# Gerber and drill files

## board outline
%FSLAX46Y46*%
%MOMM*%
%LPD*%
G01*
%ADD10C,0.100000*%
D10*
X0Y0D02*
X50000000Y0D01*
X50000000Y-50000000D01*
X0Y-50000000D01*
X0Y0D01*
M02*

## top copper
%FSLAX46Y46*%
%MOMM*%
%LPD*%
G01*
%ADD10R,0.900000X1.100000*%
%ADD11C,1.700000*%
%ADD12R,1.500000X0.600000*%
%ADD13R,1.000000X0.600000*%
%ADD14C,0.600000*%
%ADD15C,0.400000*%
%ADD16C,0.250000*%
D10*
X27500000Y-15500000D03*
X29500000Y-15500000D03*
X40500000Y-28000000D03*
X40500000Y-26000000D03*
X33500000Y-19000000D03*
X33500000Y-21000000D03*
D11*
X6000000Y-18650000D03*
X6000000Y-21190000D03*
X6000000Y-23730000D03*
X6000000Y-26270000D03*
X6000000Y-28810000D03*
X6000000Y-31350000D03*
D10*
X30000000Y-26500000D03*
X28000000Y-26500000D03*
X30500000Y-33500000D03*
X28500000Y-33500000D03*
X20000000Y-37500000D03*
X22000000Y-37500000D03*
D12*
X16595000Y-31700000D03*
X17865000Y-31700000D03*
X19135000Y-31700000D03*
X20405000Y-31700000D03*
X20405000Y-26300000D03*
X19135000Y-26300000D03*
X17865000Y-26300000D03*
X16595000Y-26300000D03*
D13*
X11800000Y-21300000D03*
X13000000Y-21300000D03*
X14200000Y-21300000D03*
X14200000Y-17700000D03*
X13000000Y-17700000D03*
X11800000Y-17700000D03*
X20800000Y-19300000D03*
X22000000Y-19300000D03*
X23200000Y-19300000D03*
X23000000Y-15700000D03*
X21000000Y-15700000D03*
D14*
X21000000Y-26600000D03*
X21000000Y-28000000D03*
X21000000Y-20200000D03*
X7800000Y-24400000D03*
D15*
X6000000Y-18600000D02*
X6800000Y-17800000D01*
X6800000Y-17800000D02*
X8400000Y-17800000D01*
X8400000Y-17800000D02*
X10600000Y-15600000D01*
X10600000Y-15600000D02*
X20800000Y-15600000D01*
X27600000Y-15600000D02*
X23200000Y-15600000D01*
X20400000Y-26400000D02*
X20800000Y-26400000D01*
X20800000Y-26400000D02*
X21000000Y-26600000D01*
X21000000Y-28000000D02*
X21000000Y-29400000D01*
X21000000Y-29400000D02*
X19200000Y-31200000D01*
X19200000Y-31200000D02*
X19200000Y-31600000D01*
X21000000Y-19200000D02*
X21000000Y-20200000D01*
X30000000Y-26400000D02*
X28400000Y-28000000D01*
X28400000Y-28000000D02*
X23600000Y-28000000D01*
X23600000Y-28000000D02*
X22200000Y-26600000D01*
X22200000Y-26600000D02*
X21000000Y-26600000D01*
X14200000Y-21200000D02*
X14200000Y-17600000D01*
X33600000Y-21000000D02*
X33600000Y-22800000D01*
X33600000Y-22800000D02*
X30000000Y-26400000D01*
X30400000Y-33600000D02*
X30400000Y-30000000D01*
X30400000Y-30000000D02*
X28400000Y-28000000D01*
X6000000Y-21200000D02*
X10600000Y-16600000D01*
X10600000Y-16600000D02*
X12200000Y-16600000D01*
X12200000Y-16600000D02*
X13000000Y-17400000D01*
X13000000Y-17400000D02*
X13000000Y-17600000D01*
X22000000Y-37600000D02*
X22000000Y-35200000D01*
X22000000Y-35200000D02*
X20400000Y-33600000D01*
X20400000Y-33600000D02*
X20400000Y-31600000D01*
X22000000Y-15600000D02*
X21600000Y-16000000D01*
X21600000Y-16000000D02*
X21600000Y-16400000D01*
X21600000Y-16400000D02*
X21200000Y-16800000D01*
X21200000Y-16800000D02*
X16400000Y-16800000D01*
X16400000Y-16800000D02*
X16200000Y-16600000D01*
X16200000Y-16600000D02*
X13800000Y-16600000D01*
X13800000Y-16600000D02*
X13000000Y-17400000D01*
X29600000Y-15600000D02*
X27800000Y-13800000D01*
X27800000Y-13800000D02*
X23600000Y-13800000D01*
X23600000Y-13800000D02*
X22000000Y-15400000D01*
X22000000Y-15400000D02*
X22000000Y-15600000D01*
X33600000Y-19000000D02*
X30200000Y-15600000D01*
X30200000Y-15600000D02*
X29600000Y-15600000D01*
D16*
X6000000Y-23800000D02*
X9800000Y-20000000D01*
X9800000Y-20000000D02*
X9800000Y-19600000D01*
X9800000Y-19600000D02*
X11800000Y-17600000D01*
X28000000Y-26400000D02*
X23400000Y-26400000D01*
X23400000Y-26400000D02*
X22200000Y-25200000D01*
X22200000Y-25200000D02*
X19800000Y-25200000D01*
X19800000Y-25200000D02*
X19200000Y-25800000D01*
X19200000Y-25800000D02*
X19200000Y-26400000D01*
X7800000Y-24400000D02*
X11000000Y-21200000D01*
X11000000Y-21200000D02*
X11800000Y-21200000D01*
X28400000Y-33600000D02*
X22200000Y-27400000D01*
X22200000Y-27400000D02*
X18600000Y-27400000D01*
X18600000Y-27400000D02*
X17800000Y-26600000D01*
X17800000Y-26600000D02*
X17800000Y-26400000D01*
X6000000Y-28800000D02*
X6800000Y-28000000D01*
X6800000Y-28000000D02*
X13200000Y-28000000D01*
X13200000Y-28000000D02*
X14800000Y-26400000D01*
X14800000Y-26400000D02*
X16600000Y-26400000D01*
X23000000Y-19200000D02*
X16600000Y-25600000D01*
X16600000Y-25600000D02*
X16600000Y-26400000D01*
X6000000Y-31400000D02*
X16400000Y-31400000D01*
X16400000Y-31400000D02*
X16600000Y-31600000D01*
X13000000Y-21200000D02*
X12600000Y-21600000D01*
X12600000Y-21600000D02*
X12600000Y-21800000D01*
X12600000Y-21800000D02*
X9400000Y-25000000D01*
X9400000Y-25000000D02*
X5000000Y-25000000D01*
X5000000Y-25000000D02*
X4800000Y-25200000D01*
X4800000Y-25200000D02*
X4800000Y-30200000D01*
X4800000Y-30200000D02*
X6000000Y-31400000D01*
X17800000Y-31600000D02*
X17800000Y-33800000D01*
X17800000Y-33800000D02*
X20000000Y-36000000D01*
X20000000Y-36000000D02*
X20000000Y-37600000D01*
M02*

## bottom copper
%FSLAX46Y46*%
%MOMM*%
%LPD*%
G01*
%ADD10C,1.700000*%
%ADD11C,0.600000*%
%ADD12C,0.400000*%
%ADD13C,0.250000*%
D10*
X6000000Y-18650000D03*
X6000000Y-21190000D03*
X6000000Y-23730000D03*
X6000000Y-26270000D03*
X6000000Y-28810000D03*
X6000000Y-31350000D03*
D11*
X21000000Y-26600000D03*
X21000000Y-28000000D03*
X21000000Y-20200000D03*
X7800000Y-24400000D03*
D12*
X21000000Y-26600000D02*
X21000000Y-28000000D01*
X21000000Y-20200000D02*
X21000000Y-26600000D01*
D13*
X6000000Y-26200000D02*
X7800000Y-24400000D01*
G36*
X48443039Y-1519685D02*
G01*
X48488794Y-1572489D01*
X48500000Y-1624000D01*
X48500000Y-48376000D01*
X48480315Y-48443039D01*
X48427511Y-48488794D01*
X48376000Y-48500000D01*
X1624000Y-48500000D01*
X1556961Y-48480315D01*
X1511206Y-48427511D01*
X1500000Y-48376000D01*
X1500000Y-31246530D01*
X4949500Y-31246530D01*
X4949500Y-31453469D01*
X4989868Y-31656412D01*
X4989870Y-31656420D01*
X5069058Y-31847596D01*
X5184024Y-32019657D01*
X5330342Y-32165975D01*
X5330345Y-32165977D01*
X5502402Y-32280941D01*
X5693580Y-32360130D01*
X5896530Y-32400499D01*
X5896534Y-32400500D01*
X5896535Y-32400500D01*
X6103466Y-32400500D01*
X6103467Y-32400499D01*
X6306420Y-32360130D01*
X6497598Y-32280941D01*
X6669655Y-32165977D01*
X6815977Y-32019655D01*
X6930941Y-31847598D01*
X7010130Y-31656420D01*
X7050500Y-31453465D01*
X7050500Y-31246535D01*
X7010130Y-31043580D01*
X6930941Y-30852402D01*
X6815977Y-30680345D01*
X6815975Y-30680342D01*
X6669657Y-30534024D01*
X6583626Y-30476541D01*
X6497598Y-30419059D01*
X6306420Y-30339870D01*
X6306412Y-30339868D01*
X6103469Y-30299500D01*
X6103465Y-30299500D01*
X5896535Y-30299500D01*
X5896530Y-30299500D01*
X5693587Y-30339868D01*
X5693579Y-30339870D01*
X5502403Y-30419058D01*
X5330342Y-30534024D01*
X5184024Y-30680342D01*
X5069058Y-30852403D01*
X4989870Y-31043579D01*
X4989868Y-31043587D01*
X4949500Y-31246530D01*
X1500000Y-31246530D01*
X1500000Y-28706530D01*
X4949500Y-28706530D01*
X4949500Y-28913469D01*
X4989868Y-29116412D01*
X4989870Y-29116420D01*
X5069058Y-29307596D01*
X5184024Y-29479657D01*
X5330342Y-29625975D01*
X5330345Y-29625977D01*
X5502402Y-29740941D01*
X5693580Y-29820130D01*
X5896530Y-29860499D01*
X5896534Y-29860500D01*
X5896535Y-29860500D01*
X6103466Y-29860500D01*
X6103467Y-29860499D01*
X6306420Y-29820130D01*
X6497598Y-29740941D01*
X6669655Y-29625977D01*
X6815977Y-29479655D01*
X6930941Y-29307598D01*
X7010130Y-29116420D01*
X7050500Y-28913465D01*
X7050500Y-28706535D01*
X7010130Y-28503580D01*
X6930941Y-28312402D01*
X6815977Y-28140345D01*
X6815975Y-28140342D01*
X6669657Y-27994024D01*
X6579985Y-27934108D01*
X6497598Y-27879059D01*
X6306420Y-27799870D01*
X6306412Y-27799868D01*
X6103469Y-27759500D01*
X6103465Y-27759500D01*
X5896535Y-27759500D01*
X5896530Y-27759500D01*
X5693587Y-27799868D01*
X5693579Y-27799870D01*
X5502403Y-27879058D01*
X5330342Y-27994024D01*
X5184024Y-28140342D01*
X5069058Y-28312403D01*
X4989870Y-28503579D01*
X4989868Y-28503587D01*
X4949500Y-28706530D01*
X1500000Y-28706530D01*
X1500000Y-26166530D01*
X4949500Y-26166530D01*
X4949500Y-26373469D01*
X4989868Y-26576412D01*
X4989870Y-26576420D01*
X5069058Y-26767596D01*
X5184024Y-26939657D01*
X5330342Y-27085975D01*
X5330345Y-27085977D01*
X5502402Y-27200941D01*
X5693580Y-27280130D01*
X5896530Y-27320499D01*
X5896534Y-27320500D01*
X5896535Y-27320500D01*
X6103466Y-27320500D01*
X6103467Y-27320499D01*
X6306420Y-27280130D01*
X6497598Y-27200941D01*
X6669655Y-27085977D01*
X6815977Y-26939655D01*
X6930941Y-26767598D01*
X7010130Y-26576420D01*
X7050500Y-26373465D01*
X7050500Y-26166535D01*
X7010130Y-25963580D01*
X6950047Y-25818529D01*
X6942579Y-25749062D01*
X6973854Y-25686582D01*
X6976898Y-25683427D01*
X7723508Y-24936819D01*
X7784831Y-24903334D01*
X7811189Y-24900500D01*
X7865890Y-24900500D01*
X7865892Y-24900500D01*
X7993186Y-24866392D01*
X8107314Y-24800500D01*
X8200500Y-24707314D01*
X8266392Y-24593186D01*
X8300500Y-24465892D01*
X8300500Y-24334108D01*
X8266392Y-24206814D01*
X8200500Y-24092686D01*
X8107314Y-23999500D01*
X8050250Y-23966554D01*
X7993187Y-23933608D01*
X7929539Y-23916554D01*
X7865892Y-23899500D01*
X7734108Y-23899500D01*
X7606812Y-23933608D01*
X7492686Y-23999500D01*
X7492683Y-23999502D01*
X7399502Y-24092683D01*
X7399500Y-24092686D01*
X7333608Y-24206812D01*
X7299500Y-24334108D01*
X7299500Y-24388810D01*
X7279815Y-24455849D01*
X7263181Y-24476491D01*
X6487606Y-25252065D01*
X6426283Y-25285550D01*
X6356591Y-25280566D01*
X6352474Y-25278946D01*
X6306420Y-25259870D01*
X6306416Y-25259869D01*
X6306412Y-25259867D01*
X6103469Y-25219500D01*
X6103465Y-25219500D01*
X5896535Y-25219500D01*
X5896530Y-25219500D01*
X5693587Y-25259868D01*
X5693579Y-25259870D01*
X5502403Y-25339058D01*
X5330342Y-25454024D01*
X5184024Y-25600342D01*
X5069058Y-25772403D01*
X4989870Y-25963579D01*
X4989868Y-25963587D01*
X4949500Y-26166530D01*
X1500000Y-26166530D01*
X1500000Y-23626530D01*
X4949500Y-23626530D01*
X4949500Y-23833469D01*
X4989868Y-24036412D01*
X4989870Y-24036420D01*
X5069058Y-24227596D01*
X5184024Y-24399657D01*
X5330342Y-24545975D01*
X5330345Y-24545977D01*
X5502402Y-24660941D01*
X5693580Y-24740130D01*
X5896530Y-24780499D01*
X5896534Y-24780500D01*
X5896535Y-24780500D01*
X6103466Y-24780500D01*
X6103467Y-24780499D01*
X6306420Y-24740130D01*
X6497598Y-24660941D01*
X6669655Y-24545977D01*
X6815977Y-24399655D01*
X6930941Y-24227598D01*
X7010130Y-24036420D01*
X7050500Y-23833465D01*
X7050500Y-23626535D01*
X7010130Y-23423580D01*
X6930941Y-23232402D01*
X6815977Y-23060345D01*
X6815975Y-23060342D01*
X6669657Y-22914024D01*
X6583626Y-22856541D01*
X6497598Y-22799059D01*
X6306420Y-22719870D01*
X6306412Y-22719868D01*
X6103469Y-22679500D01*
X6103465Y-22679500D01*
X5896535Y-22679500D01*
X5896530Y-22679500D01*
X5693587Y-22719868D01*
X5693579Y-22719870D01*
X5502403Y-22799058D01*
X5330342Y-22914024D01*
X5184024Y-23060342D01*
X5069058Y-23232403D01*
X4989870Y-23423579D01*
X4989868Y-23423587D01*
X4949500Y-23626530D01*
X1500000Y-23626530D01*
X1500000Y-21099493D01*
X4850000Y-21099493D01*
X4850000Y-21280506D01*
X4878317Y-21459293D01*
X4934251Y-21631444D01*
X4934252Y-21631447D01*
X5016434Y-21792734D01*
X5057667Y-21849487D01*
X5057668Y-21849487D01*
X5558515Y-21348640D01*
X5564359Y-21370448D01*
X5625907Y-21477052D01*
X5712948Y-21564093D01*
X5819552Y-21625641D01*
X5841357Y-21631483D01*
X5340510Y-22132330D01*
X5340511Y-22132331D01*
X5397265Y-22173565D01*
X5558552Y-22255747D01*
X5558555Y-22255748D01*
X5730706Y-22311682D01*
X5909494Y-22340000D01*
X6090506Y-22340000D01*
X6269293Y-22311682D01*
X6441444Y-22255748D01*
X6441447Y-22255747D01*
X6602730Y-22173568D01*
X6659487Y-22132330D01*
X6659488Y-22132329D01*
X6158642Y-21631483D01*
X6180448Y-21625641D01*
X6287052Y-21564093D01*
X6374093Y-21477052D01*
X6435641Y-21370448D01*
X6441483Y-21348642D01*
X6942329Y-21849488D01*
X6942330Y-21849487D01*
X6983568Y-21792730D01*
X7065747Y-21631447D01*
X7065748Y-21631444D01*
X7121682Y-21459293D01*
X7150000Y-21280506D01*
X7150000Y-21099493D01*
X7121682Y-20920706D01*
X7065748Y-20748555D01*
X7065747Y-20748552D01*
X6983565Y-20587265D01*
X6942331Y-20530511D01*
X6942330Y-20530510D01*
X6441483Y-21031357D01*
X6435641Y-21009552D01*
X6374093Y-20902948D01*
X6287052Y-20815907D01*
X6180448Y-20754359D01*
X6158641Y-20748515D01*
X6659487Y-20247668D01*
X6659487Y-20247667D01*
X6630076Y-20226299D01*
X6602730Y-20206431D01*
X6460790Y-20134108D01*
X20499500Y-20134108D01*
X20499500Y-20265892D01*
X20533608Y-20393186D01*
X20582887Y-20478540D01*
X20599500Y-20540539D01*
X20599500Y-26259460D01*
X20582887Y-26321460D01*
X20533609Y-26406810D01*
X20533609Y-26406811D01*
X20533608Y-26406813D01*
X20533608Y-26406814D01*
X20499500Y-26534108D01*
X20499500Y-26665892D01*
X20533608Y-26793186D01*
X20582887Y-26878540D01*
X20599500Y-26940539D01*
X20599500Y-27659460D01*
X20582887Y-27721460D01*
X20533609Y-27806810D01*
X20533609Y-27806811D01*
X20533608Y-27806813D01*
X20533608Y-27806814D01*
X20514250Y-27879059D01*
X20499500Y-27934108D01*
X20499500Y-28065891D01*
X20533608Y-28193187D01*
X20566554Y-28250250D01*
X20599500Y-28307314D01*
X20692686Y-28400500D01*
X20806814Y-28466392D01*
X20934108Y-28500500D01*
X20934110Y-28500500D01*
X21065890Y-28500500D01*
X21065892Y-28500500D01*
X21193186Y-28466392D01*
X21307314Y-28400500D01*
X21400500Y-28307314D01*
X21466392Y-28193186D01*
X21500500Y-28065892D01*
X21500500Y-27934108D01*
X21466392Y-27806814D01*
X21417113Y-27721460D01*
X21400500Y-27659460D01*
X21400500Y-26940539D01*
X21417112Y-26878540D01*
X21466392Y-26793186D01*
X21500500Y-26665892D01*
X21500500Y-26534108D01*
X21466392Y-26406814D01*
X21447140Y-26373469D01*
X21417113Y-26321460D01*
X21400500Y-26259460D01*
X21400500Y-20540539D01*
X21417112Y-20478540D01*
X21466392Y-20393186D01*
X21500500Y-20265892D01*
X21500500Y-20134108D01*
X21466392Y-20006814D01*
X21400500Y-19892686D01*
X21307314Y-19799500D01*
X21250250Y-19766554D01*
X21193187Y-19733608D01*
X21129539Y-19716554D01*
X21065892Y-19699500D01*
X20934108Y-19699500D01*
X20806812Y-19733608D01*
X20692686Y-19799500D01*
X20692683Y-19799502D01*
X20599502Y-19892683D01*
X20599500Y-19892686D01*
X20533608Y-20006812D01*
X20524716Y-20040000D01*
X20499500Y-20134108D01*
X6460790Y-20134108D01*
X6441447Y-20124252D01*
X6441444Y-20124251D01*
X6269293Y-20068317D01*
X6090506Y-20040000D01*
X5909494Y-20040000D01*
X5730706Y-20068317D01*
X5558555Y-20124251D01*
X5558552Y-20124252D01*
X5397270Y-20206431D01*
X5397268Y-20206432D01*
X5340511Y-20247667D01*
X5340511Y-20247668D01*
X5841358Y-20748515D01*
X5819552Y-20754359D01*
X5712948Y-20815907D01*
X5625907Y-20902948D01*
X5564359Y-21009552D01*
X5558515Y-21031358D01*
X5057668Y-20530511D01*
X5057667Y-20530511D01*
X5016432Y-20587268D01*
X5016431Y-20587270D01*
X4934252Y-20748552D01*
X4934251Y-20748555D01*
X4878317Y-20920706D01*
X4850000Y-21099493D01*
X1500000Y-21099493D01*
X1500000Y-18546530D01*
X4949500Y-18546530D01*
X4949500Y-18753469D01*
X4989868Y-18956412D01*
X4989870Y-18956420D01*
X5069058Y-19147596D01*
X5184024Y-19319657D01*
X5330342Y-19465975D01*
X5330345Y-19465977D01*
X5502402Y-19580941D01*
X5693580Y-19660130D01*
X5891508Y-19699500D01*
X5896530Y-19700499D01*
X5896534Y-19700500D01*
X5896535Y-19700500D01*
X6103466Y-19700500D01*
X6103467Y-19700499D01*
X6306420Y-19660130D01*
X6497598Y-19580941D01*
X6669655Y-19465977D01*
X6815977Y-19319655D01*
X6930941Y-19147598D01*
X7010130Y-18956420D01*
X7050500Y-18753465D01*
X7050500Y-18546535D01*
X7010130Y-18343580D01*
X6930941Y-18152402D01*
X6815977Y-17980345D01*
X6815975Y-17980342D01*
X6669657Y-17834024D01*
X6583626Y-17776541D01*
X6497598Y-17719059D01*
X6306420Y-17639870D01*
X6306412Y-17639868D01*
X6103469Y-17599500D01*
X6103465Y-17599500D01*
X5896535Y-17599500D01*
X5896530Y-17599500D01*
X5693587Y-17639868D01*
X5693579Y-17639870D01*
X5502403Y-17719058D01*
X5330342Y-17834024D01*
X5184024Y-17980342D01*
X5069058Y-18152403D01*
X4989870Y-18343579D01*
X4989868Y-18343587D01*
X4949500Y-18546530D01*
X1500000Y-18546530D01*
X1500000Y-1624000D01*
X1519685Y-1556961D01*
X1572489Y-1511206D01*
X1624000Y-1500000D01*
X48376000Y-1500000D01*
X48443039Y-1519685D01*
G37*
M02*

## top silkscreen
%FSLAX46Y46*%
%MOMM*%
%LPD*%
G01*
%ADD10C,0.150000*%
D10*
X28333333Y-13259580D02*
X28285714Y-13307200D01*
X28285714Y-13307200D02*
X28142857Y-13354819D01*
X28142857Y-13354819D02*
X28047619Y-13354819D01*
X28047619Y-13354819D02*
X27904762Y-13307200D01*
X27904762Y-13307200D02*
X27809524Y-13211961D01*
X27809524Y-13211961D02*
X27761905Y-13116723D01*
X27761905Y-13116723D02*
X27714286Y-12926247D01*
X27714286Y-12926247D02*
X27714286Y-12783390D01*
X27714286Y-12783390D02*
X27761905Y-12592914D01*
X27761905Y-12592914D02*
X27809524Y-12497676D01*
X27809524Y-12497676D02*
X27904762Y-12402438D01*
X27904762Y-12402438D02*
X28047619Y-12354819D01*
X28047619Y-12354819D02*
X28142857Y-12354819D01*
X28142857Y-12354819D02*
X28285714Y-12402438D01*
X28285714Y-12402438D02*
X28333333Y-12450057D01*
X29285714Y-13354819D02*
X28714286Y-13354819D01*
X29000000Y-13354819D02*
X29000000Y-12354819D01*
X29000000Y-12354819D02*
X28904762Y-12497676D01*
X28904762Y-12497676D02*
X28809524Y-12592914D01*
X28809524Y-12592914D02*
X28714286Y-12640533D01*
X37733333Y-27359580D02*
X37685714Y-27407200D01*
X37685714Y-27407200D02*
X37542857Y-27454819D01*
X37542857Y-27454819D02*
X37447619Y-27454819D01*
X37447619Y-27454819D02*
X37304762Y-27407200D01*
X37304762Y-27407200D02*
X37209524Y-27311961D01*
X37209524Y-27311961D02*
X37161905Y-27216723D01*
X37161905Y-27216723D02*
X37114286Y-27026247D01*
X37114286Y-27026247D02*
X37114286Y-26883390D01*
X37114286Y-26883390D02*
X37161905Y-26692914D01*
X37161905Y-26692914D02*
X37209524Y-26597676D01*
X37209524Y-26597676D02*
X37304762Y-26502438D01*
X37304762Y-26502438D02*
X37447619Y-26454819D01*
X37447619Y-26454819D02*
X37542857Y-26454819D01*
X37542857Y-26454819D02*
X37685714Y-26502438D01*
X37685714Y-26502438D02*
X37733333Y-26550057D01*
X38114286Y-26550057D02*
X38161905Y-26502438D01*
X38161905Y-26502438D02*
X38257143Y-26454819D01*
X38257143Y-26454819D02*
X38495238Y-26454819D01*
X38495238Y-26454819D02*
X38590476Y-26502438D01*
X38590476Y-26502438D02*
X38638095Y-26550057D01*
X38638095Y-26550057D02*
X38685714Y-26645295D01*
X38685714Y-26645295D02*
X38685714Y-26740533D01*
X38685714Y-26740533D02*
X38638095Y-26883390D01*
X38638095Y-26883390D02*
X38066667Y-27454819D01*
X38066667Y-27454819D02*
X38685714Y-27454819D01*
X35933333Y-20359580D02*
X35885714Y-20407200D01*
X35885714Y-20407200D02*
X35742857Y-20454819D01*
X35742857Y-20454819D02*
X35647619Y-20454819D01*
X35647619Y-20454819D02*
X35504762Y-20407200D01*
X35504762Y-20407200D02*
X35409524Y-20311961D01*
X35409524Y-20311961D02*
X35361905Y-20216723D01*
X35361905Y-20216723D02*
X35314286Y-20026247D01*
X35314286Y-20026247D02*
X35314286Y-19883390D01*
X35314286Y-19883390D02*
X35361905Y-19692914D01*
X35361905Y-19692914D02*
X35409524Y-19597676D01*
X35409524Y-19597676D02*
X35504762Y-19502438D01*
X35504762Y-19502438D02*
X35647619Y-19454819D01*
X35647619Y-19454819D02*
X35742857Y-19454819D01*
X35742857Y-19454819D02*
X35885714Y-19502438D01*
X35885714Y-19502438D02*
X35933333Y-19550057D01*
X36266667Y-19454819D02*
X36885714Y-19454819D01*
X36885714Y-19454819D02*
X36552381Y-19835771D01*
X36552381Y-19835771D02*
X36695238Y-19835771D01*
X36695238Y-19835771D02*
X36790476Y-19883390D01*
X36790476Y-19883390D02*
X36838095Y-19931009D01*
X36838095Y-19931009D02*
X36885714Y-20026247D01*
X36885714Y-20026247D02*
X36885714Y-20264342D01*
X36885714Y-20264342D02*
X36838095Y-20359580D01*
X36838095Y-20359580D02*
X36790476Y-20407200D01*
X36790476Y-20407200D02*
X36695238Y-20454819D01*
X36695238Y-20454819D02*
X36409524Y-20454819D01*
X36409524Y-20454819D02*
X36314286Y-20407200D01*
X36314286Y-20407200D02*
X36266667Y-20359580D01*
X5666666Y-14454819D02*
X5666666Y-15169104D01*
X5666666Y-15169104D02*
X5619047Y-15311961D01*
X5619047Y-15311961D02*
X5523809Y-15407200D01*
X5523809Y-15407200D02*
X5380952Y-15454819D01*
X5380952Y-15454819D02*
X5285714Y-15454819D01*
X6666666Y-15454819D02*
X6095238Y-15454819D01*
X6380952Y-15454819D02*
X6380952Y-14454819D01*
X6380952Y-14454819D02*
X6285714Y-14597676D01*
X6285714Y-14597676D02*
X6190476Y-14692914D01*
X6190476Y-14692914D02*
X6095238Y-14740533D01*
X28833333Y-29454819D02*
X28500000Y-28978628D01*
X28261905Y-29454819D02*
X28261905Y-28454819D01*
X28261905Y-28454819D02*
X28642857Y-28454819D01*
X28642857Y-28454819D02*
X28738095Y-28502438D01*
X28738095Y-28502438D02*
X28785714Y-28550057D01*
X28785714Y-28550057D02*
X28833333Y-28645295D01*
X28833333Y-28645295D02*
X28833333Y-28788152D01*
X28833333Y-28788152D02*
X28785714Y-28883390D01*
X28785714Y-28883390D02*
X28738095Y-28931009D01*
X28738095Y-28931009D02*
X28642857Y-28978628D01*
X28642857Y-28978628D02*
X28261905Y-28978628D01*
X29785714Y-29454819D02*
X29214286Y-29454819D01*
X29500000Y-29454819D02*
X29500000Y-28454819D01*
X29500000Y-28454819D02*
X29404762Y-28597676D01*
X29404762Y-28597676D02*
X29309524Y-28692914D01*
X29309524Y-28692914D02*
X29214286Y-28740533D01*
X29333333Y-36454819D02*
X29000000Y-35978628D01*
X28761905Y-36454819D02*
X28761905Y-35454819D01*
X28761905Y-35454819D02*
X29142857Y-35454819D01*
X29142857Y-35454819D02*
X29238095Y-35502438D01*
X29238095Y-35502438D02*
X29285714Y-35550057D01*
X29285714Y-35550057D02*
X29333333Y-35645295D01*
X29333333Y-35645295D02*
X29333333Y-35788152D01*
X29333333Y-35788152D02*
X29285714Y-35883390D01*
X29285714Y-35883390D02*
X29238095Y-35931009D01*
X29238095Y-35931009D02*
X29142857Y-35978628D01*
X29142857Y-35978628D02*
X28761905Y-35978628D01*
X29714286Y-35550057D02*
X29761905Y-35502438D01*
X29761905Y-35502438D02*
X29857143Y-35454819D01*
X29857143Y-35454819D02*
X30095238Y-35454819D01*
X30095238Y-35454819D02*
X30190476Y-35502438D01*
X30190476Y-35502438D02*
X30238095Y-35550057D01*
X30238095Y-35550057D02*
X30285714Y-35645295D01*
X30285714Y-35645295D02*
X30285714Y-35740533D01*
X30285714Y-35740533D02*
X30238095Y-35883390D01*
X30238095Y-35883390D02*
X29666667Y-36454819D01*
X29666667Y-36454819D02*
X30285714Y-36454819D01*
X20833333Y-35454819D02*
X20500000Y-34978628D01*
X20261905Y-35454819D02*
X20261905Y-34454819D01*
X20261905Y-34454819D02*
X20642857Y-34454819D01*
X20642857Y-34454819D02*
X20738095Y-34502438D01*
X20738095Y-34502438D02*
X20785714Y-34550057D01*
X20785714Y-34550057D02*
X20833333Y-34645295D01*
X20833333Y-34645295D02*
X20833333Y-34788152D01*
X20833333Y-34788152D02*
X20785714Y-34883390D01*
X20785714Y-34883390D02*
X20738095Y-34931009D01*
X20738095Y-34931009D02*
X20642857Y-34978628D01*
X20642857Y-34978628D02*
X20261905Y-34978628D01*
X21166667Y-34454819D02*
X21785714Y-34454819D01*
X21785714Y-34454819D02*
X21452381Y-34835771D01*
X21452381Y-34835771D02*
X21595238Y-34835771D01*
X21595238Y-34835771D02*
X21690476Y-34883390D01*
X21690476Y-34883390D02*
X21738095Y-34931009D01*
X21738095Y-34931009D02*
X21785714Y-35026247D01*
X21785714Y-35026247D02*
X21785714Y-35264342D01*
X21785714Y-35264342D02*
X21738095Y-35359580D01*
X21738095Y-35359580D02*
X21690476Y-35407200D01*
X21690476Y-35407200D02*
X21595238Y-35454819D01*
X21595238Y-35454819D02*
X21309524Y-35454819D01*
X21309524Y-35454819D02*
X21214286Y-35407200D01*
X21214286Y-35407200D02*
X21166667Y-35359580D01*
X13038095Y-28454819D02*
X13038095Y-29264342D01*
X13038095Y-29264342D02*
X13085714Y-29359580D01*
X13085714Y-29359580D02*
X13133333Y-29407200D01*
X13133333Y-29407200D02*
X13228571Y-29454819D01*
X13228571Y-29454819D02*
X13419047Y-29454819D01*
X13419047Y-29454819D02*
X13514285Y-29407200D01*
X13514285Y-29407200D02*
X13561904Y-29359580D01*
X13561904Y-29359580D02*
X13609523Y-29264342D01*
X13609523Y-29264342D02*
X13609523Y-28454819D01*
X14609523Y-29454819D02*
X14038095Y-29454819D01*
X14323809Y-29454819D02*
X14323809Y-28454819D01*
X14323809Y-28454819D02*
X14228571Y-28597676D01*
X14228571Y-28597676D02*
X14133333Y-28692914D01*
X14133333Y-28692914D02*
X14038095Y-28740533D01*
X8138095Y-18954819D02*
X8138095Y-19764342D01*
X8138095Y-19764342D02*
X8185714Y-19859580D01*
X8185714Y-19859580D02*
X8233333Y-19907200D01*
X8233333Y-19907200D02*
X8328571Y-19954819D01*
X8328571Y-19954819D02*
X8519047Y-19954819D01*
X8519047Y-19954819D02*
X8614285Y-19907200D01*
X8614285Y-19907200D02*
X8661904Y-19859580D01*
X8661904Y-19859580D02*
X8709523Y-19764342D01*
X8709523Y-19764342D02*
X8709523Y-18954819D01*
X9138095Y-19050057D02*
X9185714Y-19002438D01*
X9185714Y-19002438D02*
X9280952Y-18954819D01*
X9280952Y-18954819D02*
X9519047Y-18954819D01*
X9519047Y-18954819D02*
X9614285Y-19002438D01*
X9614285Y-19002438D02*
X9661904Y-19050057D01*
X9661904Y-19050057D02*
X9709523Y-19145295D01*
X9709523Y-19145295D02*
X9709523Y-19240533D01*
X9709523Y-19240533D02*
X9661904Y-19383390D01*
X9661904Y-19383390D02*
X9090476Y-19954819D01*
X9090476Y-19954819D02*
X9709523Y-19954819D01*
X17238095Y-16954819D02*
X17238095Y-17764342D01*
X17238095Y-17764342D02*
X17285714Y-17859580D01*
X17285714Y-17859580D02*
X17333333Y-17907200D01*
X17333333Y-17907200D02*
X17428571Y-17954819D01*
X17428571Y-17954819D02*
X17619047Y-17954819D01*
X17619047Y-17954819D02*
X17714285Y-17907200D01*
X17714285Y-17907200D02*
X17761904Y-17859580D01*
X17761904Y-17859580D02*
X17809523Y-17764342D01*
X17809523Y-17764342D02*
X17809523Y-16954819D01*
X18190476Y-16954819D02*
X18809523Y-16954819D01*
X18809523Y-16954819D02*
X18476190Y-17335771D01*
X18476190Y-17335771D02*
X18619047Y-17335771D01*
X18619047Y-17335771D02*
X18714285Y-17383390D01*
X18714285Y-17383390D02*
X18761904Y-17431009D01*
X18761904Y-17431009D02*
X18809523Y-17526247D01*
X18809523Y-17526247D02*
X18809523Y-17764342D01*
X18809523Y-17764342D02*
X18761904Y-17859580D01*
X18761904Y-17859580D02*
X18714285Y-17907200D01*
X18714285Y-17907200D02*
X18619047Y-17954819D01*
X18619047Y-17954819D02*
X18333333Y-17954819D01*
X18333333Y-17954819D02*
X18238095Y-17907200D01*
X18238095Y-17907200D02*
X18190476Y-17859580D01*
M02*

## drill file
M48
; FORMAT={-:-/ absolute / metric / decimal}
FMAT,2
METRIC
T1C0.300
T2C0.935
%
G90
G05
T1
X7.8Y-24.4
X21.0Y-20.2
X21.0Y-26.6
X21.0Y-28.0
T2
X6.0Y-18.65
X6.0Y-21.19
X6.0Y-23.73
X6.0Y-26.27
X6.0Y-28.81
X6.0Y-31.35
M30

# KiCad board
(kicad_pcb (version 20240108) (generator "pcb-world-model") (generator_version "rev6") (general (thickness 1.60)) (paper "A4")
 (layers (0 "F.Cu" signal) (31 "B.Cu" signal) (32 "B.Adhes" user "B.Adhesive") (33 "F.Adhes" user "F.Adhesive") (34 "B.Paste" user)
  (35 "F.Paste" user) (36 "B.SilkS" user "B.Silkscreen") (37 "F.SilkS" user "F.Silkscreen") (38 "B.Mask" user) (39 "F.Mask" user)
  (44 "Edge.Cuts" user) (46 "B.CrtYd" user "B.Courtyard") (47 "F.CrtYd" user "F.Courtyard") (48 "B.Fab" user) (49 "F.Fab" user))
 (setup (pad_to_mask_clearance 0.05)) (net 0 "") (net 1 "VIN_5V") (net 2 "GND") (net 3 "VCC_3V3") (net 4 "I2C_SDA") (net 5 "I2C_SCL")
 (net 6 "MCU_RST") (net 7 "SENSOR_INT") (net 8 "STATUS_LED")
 (gr_rect (start 0.0 0.0) (end 50.0000 50.0000) (stroke (width 0.1) (type default)) (fill none) (layer "Edge.Cuts"))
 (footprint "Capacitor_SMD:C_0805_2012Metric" (layer "F.Cu") (at 28.5000 15.5000 0)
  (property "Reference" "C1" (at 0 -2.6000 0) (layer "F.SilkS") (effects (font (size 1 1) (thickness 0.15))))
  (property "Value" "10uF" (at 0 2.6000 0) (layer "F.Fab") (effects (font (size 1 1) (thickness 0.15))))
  (pad "1" smd rect (at -1.0000 0.0000) (size 0.9000 1.1000) (layers "F.Cu" "F.Paste" "F.Mask") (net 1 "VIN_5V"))
  (pad "2" smd rect (at 1.0000 0.0000) (size 0.9000 1.1000) (layers "F.Cu" "F.Paste" "F.Mask") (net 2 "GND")))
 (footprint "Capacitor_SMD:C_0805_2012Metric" (layer "F.Cu") (at 40.5000 27.0000 90)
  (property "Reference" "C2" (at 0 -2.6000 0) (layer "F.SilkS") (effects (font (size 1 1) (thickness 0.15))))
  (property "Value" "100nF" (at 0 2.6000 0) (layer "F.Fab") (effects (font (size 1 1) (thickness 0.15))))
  (pad "1" smd rect (at -1.0000 0.0000) (size 0.9000 1.1000) (layers "F.Cu" "F.Paste" "F.Mask") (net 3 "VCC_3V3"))
  (pad "2" smd rect (at 1.0000 0.0000) (size 0.9000 1.1000) (layers "F.Cu" "F.Paste" "F.Mask") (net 2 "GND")))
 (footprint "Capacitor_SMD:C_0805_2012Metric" (layer "F.Cu") (at 33.5000 20.0000 270)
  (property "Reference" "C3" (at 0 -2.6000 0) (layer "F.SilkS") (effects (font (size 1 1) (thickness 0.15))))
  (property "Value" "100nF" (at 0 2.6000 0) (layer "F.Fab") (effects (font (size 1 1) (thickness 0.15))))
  (pad "1" smd rect (at -1.0000 0.0000) (size 0.9000 1.1000) (layers "F.Cu" "F.Paste" "F.Mask") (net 3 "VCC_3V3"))
  (pad "2" smd rect (at 1.0000 0.0000) (size 0.9000 1.1000) (layers "F.Cu" "F.Paste" "F.Mask") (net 2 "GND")))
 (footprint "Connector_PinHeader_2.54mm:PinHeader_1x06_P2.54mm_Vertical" (layer "F.Cu") (at 6.0000 25.0000 0) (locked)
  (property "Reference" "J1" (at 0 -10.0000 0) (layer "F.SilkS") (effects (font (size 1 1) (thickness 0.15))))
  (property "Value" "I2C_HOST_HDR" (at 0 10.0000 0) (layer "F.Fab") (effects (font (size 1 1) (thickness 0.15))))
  (pad "1" thru_hole circle (at 0.0000 -6.3500) (size 1.7000 1.7000) (drill 0.9350) (layers "*.Cu" "*.Mask") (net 1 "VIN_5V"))
  (pad "2" thru_hole circle (at 0.0000 -3.8100) (size 1.7000 1.7000) (drill 0.9350) (layers "*.Cu" "*.Mask") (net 2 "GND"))
  (pad "3" thru_hole circle (at 0.0000 -1.2700) (size 1.7000 1.7000) (drill 0.9350) (layers "*.Cu" "*.Mask") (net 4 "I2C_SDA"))
  (pad "4" thru_hole circle (at 0.0000 1.2700) (size 1.7000 1.7000) (drill 0.9350) (layers "*.Cu" "*.Mask") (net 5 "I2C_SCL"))
  (pad "5" thru_hole circle (at 0.0000 3.8100) (size 1.7000 1.7000) (drill 0.9350) (layers "*.Cu" "*.Mask") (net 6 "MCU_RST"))
  (pad "6" thru_hole circle (at 0.0000 6.3500) (size 1.7000 1.7000) (drill 0.9350) (layers "*.Cu" "*.Mask") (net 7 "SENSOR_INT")))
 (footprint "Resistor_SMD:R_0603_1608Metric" (layer "F.Cu") (at 29.0000 26.5000 180)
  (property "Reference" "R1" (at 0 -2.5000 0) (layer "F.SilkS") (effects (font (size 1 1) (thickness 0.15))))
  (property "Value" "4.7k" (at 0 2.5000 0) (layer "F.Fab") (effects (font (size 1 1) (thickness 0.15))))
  (pad "1" smd rect (at -1.0000 0.0000) (size 0.9000 1.1000) (layers "F.Cu" "F.Paste" "F.Mask") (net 3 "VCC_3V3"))
  (pad "2" smd rect (at 1.0000 0.0000) (size 0.9000 1.1000) (layers "F.Cu" "F.Paste" "F.Mask") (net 4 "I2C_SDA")))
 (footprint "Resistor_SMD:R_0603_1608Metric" (layer "F.Cu") (at 29.5000 33.5000 180)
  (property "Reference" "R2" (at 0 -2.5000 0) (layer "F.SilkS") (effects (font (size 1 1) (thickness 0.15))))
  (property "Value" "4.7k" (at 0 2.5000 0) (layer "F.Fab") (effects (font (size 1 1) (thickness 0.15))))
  (pad "1" smd rect (at -1.0000 0.0000) (size 0.9000 1.1000) (layers "F.Cu" "F.Paste" "F.Mask") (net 3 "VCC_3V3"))
  (pad "2" smd rect (at 1.0000 0.0000) (size 0.9000 1.1000) (layers "F.Cu" "F.Paste" "F.Mask") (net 5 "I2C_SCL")))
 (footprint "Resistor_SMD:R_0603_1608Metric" (layer "F.Cu") (at 21.0000 37.5000 0)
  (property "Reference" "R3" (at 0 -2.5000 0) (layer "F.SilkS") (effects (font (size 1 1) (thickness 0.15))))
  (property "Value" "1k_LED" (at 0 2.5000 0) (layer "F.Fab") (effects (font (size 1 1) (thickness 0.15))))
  (pad "1" smd rect (at -1.0000 0.0000) (size 0.9000 1.1000) (layers "F.Cu" "F.Paste" "F.Mask") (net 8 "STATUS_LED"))
  (pad "2" smd rect (at 1.0000 0.0000) (size 0.9000 1.1000) (layers "F.Cu" "F.Paste" "F.Mask") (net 2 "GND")))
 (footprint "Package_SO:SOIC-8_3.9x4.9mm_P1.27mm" (layer "F.Cu") (at 18.5000 29.0000 90)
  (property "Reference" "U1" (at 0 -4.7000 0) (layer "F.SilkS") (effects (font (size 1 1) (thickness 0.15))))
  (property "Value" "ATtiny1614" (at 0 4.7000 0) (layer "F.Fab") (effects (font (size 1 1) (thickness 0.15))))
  (pad "1" smd rect (at -2.7000 -1.9050) (size 1.5000 0.6000) (layers "F.Cu" "F.Paste" "F.Mask") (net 3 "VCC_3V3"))
  (pad "2" smd rect (at -2.7000 -0.6350) (size 1.5000 0.6000) (layers "F.Cu" "F.Paste" "F.Mask") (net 4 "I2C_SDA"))
  (pad "3" smd rect (at -2.7000 0.6350) (size 1.5000 0.6000) (layers "F.Cu" "F.Paste" "F.Mask") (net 5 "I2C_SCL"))
  (pad "4" smd rect (at -2.7000 1.9050) (size 1.5000 0.6000) (layers "F.Cu" "F.Paste" "F.Mask") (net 6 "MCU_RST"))
  (pad "5" smd rect (at 2.7000 1.9050) (size 1.5000 0.6000) (layers "F.Cu" "F.Paste" "F.Mask") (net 7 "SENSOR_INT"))
  (pad "6" smd rect (at 2.7000 0.6350) (size 1.5000 0.6000) (layers "F.Cu" "F.Paste" "F.Mask") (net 8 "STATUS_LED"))
  (pad "7" smd rect (at 2.7000 -0.6350) (size 1.5000 0.6000) (layers "F.Cu" "F.Paste" "F.Mask") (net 3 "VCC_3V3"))
  (pad "8" smd rect (at 2.7000 -1.9050) (size 1.5000 0.6000) (layers "F.Cu" "F.Paste" "F.Mask") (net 2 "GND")))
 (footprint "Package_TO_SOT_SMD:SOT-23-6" (layer "F.Cu") (at 13.0000 19.5000 90)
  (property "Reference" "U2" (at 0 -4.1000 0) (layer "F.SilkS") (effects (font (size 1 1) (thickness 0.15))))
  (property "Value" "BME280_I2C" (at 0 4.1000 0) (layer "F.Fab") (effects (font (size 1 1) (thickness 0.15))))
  (pad "1" smd rect (at -1.8000 -1.2000) (size 1.0000 0.6000) (layers "F.Cu" "F.Paste" "F.Mask") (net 3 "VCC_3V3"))
  (pad "2" smd rect (at -1.8000 0.0000) (size 1.0000 0.6000) (layers "F.Cu" "F.Paste" "F.Mask") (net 2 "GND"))
  (pad "3" smd rect (at -1.8000 1.2000) (size 1.0000 0.6000) (layers "F.Cu" "F.Paste" "F.Mask") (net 4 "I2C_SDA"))
  (pad "4" smd rect (at 1.8000 1.2000) (size 1.0000 0.6000) (layers "F.Cu" "F.Paste" "F.Mask") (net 5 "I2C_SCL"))
  (pad "5" smd rect (at 1.8000 0.0000) (size 1.0000 0.6000) (layers "F.Cu" "F.Paste" "F.Mask") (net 7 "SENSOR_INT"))
  (pad "6" smd rect (at 1.8000 -1.2000) (size 1.0000 0.6000) (layers "F.Cu" "F.Paste" "F.Mask") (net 3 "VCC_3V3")))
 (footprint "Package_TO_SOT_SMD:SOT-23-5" (layer "F.Cu") (at 22.0000 17.5000 90)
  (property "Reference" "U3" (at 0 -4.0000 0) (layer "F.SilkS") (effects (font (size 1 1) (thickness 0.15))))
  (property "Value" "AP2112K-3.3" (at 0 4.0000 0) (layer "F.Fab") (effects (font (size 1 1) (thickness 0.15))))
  (pad "1" smd rect (at -1.8000 -1.2000) (size 1.0000 0.6000) (layers "F.Cu" "F.Paste" "F.Mask") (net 1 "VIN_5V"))
  (pad "2" smd rect (at -1.8000 0.0000) (size 1.0000 0.6000) (layers "F.Cu" "F.Paste" "F.Mask") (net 2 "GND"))
  (pad "3" smd rect (at -1.8000 1.2000) (size 1.0000 0.6000) (layers "F.Cu" "F.Paste" "F.Mask") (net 1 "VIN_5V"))
  (pad "4" smd rect (at 1.8000 1.0000) (size 1.0000 0.6000) (layers "F.Cu" "F.Paste" "F.Mask") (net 3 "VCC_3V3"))
  (pad "5" smd rect (at 1.8000 -1.0000) (size 1.0000 0.6000) (layers "F.Cu" "F.Paste" "F.Mask") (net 6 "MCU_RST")))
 (segment (start 6.0000 18.6000) (end 6.8000 17.8000) (width 0.4000) (layer "F.Cu") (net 1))
 (segment (start 6.8000 17.8000) (end 8.4000 17.8000) (width 0.4000) (layer "F.Cu") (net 1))
 (segment (start 8.4000 17.8000) (end 10.6000 15.6000) (width 0.4000) (layer "F.Cu") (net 1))
 (segment (start 10.6000 15.6000) (end 20.8000 15.6000) (width 0.4000) (layer "F.Cu") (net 1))
 (segment (start 27.6000 15.6000) (end 23.2000 15.6000) (width 0.4000) (layer "F.Cu") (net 1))
 (segment (start 20.4000 26.4000) (end 20.8000 26.4000) (width 0.4000) (layer "F.Cu") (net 3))
 (segment (start 20.8000 26.4000) (end 21.0000 26.6000) (width 0.4000) (layer "F.Cu") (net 3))
 (segment (start 21.0000 26.6000) (end 21.0000 28.0000) (width 0.4000) (layer "B.Cu") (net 3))
 (segment (start 21.0000 28.0000) (end 21.0000 29.4000) (width 0.4000) (layer "F.Cu") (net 3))
 (segment (start 21.0000 29.4000) (end 19.2000 31.2000) (width 0.4000) (layer "F.Cu") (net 3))
 (segment (start 19.2000 31.2000) (end 19.2000 31.6000) (width 0.4000) (layer "F.Cu") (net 3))
 (segment (start 21.0000 19.2000) (end 21.0000 20.2000) (width 0.4000) (layer "F.Cu") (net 3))
 (segment (start 21.0000 20.2000) (end 21.0000 26.6000) (width 0.4000) (layer "B.Cu") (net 3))
 (segment (start 30.0000 26.4000) (end 28.4000 28.0000) (width 0.4000) (layer "F.Cu") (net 3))
 (segment (start 28.4000 28.0000) (end 23.6000 28.0000) (width 0.4000) (layer "F.Cu") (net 3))
 (segment (start 23.6000 28.0000) (end 22.2000 26.6000) (width 0.4000) (layer "F.Cu") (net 3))
 (segment (start 22.2000 26.6000) (end 21.0000 26.6000) (width 0.4000) (layer "F.Cu") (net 3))
 (segment (start 14.2000 21.2000) (end 14.2000 17.6000) (width 0.4000) (layer "F.Cu") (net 3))
 (segment (start 33.6000 21.0000) (end 33.6000 22.8000) (width 0.4000) (layer "F.Cu") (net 3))
 (segment (start 33.6000 22.8000) (end 30.0000 26.4000) (width 0.4000) (layer "F.Cu") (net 3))
 (segment (start 30.4000 33.6000) (end 30.4000 30.0000) (width 0.4000) (layer "F.Cu") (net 3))
 (segment (start 30.4000 30.0000) (end 28.4000 28.0000) (width 0.4000) (layer "F.Cu") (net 3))
 (segment (start 6.0000 21.2000) (end 10.6000 16.6000) (width 0.4000) (layer "F.Cu") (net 2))
 (segment (start 10.6000 16.6000) (end 12.2000 16.6000) (width 0.4000) (layer "F.Cu") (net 2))
 (segment (start 12.2000 16.6000) (end 13.0000 17.4000) (width 0.4000) (layer "F.Cu") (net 2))
 (segment (start 13.0000 17.4000) (end 13.0000 17.6000) (width 0.4000) (layer "F.Cu") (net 2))
 (segment (start 22.0000 37.6000) (end 22.0000 35.2000) (width 0.4000) (layer "F.Cu") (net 2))
 (segment (start 22.0000 35.2000) (end 20.4000 33.6000) (width 0.4000) (layer "F.Cu") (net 2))
 (segment (start 20.4000 33.6000) (end 20.4000 31.6000) (width 0.4000) (layer "F.Cu") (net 2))
 (segment (start 22.0000 15.6000) (end 21.6000 16.0000) (width 0.4000) (layer "F.Cu") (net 2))
 (segment (start 21.6000 16.0000) (end 21.6000 16.4000) (width 0.4000) (layer "F.Cu") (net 2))
 (segment (start 21.6000 16.4000) (end 21.2000 16.8000) (width 0.4000) (layer "F.Cu") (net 2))
 (segment (start 21.2000 16.8000) (end 16.4000 16.8000) (width 0.4000) (layer "F.Cu") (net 2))
 (segment (start 16.4000 16.8000) (end 16.2000 16.6000) (width 0.4000) (layer "F.Cu") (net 2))
 (segment (start 16.2000 16.6000) (end 13.8000 16.6000) (width 0.4000) (layer "F.Cu") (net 2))
 (segment (start 13.8000 16.6000) (end 13.0000 17.4000) (width 0.4000) (layer "F.Cu") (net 2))
 (segment (start 29.6000 15.6000) (end 27.8000 13.8000) (width 0.4000) (layer "F.Cu") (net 2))
 (segment (start 27.8000 13.8000) (end 23.6000 13.8000) (width 0.4000) (layer "F.Cu") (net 2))
 (segment (start 23.6000 13.8000) (end 22.0000 15.4000) (width 0.4000) (layer "F.Cu") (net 2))
 (segment (start 22.0000 15.4000) (end 22.0000 15.6000) (width 0.4000) (layer "F.Cu") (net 2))
 (segment (start 33.6000 19.0000) (end 30.2000 15.6000) (width 0.4000) (layer "F.Cu") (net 2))
 (segment (start 30.2000 15.6000) (end 29.6000 15.6000) (width 0.4000) (layer "F.Cu") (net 2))
 (segment (start 6.0000 23.8000) (end 9.8000 20.0000) (width 0.2500) (layer "F.Cu") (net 4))
 (segment (start 9.8000 20.0000) (end 9.8000 19.6000) (width 0.2500) (layer "F.Cu") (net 4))
 (segment (start 9.8000 19.6000) (end 11.8000 17.6000) (width 0.2500) (layer "F.Cu") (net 4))
 (segment (start 28.0000 26.4000) (end 23.4000 26.4000) (width 0.2500) (layer "F.Cu") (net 4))
 (segment (start 23.4000 26.4000) (end 22.2000 25.2000) (width 0.2500) (layer "F.Cu") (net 4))
 (segment (start 22.2000 25.2000) (end 19.8000 25.2000) (width 0.2500) (layer "F.Cu") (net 4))
 (segment (start 19.8000 25.2000) (end 19.2000 25.8000) (width 0.2500) (layer "F.Cu") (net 4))
 (segment (start 19.2000 25.8000) (end 19.2000 26.4000) (width 0.2500) (layer "F.Cu") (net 4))
 (segment (start 6.0000 26.2000) (end 7.8000 24.4000) (width 0.2500) (layer "B.Cu") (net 5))
 (segment (start 7.8000 24.4000) (end 11.0000 21.2000) (width 0.2500) (layer "F.Cu") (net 5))
 (segment (start 11.0000 21.2000) (end 11.8000 21.2000) (width 0.2500) (layer "F.Cu") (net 5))
 (segment (start 28.4000 33.6000) (end 22.2000 27.4000) (width 0.2500) (layer "F.Cu") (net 5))
 (segment (start 22.2000 27.4000) (end 18.6000 27.4000) (width 0.2500) (layer "F.Cu") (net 5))
 (segment (start 18.6000 27.4000) (end 17.8000 26.6000) (width 0.2500) (layer "F.Cu") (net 5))
 (segment (start 17.8000 26.6000) (end 17.8000 26.4000) (width 0.2500) (layer "F.Cu") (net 5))
 (segment (start 6.0000 28.8000) (end 6.8000 28.0000) (width 0.2500) (layer "F.Cu") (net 6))
 (segment (start 6.8000 28.0000) (end 13.2000 28.0000) (width 0.2500) (layer "F.Cu") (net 6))
 (segment (start 13.2000 28.0000) (end 14.8000 26.4000) (width 0.2500) (layer "F.Cu") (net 6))
 (segment (start 14.8000 26.4000) (end 16.6000 26.4000) (width 0.2500) (layer "F.Cu") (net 6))
 (segment (start 23.0000 19.2000) (end 16.6000 25.6000) (width 0.2500) (layer "F.Cu") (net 6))
 (segment (start 16.6000 25.6000) (end 16.6000 26.4000) (width 0.2500) (layer "F.Cu") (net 6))
 (segment (start 6.0000 31.4000) (end 16.4000 31.4000) (width 0.2500) (layer "F.Cu") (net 7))
 (segment (start 16.4000 31.4000) (end 16.6000 31.6000) (width 0.2500) (layer "F.Cu") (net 7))
 (segment (start 13.0000 21.2000) (end 12.6000 21.6000) (width 0.2500) (layer "F.Cu") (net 7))
 (segment (start 12.6000 21.6000) (end 12.6000 21.8000) (width 0.2500) (layer "F.Cu") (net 7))
 (segment (start 12.6000 21.8000) (end 9.4000 25.0000) (width 0.2500) (layer "F.Cu") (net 7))
 (segment (start 9.4000 25.0000) (end 5.0000 25.0000) (width 0.2500) (layer "F.Cu") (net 7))
 (segment (start 5.0000 25.0000) (end 4.8000 25.2000) (width 0.2500) (layer "F.Cu") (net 7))
 (segment (start 4.8000 25.2000) (end 4.8000 30.2000) (width 0.2500) (layer "F.Cu") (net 7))
 (segment (start 4.8000 30.2000) (end 6.0000 31.4000) (width 0.2500) (layer "F.Cu") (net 7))
 (segment (start 17.8000 31.6000) (end 17.8000 33.8000) (width 0.2500) (layer "F.Cu") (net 8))
 (segment (start 17.8000 33.8000) (end 20.0000 36.0000) (width 0.2500) (layer "F.Cu") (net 8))
 (segment (start 20.0000 36.0000) (end 20.0000 37.6000) (width 0.2500) (layer "F.Cu") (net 8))
 (via (at 21.0000 26.6000) (size 0.6000) (drill 0.3000) (layers "F.Cu" "B.Cu") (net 3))
 (via (at 21.0000 28.0000) (size 0.6000) (drill 0.3000) (layers "F.Cu" "B.Cu") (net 3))
 (via (at 21.0000 20.2000) (size 0.6000) (drill 0.3000) (layers "F.Cu" "B.Cu") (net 3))
 (via (at 7.8000 24.4000) (size 0.6000) (drill 0.3000) (layers "F.Cu" "B.Cu") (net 5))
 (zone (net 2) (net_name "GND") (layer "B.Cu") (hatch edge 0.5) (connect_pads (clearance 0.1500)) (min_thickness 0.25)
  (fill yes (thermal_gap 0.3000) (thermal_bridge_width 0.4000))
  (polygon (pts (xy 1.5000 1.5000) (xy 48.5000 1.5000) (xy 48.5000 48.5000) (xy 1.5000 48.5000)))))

